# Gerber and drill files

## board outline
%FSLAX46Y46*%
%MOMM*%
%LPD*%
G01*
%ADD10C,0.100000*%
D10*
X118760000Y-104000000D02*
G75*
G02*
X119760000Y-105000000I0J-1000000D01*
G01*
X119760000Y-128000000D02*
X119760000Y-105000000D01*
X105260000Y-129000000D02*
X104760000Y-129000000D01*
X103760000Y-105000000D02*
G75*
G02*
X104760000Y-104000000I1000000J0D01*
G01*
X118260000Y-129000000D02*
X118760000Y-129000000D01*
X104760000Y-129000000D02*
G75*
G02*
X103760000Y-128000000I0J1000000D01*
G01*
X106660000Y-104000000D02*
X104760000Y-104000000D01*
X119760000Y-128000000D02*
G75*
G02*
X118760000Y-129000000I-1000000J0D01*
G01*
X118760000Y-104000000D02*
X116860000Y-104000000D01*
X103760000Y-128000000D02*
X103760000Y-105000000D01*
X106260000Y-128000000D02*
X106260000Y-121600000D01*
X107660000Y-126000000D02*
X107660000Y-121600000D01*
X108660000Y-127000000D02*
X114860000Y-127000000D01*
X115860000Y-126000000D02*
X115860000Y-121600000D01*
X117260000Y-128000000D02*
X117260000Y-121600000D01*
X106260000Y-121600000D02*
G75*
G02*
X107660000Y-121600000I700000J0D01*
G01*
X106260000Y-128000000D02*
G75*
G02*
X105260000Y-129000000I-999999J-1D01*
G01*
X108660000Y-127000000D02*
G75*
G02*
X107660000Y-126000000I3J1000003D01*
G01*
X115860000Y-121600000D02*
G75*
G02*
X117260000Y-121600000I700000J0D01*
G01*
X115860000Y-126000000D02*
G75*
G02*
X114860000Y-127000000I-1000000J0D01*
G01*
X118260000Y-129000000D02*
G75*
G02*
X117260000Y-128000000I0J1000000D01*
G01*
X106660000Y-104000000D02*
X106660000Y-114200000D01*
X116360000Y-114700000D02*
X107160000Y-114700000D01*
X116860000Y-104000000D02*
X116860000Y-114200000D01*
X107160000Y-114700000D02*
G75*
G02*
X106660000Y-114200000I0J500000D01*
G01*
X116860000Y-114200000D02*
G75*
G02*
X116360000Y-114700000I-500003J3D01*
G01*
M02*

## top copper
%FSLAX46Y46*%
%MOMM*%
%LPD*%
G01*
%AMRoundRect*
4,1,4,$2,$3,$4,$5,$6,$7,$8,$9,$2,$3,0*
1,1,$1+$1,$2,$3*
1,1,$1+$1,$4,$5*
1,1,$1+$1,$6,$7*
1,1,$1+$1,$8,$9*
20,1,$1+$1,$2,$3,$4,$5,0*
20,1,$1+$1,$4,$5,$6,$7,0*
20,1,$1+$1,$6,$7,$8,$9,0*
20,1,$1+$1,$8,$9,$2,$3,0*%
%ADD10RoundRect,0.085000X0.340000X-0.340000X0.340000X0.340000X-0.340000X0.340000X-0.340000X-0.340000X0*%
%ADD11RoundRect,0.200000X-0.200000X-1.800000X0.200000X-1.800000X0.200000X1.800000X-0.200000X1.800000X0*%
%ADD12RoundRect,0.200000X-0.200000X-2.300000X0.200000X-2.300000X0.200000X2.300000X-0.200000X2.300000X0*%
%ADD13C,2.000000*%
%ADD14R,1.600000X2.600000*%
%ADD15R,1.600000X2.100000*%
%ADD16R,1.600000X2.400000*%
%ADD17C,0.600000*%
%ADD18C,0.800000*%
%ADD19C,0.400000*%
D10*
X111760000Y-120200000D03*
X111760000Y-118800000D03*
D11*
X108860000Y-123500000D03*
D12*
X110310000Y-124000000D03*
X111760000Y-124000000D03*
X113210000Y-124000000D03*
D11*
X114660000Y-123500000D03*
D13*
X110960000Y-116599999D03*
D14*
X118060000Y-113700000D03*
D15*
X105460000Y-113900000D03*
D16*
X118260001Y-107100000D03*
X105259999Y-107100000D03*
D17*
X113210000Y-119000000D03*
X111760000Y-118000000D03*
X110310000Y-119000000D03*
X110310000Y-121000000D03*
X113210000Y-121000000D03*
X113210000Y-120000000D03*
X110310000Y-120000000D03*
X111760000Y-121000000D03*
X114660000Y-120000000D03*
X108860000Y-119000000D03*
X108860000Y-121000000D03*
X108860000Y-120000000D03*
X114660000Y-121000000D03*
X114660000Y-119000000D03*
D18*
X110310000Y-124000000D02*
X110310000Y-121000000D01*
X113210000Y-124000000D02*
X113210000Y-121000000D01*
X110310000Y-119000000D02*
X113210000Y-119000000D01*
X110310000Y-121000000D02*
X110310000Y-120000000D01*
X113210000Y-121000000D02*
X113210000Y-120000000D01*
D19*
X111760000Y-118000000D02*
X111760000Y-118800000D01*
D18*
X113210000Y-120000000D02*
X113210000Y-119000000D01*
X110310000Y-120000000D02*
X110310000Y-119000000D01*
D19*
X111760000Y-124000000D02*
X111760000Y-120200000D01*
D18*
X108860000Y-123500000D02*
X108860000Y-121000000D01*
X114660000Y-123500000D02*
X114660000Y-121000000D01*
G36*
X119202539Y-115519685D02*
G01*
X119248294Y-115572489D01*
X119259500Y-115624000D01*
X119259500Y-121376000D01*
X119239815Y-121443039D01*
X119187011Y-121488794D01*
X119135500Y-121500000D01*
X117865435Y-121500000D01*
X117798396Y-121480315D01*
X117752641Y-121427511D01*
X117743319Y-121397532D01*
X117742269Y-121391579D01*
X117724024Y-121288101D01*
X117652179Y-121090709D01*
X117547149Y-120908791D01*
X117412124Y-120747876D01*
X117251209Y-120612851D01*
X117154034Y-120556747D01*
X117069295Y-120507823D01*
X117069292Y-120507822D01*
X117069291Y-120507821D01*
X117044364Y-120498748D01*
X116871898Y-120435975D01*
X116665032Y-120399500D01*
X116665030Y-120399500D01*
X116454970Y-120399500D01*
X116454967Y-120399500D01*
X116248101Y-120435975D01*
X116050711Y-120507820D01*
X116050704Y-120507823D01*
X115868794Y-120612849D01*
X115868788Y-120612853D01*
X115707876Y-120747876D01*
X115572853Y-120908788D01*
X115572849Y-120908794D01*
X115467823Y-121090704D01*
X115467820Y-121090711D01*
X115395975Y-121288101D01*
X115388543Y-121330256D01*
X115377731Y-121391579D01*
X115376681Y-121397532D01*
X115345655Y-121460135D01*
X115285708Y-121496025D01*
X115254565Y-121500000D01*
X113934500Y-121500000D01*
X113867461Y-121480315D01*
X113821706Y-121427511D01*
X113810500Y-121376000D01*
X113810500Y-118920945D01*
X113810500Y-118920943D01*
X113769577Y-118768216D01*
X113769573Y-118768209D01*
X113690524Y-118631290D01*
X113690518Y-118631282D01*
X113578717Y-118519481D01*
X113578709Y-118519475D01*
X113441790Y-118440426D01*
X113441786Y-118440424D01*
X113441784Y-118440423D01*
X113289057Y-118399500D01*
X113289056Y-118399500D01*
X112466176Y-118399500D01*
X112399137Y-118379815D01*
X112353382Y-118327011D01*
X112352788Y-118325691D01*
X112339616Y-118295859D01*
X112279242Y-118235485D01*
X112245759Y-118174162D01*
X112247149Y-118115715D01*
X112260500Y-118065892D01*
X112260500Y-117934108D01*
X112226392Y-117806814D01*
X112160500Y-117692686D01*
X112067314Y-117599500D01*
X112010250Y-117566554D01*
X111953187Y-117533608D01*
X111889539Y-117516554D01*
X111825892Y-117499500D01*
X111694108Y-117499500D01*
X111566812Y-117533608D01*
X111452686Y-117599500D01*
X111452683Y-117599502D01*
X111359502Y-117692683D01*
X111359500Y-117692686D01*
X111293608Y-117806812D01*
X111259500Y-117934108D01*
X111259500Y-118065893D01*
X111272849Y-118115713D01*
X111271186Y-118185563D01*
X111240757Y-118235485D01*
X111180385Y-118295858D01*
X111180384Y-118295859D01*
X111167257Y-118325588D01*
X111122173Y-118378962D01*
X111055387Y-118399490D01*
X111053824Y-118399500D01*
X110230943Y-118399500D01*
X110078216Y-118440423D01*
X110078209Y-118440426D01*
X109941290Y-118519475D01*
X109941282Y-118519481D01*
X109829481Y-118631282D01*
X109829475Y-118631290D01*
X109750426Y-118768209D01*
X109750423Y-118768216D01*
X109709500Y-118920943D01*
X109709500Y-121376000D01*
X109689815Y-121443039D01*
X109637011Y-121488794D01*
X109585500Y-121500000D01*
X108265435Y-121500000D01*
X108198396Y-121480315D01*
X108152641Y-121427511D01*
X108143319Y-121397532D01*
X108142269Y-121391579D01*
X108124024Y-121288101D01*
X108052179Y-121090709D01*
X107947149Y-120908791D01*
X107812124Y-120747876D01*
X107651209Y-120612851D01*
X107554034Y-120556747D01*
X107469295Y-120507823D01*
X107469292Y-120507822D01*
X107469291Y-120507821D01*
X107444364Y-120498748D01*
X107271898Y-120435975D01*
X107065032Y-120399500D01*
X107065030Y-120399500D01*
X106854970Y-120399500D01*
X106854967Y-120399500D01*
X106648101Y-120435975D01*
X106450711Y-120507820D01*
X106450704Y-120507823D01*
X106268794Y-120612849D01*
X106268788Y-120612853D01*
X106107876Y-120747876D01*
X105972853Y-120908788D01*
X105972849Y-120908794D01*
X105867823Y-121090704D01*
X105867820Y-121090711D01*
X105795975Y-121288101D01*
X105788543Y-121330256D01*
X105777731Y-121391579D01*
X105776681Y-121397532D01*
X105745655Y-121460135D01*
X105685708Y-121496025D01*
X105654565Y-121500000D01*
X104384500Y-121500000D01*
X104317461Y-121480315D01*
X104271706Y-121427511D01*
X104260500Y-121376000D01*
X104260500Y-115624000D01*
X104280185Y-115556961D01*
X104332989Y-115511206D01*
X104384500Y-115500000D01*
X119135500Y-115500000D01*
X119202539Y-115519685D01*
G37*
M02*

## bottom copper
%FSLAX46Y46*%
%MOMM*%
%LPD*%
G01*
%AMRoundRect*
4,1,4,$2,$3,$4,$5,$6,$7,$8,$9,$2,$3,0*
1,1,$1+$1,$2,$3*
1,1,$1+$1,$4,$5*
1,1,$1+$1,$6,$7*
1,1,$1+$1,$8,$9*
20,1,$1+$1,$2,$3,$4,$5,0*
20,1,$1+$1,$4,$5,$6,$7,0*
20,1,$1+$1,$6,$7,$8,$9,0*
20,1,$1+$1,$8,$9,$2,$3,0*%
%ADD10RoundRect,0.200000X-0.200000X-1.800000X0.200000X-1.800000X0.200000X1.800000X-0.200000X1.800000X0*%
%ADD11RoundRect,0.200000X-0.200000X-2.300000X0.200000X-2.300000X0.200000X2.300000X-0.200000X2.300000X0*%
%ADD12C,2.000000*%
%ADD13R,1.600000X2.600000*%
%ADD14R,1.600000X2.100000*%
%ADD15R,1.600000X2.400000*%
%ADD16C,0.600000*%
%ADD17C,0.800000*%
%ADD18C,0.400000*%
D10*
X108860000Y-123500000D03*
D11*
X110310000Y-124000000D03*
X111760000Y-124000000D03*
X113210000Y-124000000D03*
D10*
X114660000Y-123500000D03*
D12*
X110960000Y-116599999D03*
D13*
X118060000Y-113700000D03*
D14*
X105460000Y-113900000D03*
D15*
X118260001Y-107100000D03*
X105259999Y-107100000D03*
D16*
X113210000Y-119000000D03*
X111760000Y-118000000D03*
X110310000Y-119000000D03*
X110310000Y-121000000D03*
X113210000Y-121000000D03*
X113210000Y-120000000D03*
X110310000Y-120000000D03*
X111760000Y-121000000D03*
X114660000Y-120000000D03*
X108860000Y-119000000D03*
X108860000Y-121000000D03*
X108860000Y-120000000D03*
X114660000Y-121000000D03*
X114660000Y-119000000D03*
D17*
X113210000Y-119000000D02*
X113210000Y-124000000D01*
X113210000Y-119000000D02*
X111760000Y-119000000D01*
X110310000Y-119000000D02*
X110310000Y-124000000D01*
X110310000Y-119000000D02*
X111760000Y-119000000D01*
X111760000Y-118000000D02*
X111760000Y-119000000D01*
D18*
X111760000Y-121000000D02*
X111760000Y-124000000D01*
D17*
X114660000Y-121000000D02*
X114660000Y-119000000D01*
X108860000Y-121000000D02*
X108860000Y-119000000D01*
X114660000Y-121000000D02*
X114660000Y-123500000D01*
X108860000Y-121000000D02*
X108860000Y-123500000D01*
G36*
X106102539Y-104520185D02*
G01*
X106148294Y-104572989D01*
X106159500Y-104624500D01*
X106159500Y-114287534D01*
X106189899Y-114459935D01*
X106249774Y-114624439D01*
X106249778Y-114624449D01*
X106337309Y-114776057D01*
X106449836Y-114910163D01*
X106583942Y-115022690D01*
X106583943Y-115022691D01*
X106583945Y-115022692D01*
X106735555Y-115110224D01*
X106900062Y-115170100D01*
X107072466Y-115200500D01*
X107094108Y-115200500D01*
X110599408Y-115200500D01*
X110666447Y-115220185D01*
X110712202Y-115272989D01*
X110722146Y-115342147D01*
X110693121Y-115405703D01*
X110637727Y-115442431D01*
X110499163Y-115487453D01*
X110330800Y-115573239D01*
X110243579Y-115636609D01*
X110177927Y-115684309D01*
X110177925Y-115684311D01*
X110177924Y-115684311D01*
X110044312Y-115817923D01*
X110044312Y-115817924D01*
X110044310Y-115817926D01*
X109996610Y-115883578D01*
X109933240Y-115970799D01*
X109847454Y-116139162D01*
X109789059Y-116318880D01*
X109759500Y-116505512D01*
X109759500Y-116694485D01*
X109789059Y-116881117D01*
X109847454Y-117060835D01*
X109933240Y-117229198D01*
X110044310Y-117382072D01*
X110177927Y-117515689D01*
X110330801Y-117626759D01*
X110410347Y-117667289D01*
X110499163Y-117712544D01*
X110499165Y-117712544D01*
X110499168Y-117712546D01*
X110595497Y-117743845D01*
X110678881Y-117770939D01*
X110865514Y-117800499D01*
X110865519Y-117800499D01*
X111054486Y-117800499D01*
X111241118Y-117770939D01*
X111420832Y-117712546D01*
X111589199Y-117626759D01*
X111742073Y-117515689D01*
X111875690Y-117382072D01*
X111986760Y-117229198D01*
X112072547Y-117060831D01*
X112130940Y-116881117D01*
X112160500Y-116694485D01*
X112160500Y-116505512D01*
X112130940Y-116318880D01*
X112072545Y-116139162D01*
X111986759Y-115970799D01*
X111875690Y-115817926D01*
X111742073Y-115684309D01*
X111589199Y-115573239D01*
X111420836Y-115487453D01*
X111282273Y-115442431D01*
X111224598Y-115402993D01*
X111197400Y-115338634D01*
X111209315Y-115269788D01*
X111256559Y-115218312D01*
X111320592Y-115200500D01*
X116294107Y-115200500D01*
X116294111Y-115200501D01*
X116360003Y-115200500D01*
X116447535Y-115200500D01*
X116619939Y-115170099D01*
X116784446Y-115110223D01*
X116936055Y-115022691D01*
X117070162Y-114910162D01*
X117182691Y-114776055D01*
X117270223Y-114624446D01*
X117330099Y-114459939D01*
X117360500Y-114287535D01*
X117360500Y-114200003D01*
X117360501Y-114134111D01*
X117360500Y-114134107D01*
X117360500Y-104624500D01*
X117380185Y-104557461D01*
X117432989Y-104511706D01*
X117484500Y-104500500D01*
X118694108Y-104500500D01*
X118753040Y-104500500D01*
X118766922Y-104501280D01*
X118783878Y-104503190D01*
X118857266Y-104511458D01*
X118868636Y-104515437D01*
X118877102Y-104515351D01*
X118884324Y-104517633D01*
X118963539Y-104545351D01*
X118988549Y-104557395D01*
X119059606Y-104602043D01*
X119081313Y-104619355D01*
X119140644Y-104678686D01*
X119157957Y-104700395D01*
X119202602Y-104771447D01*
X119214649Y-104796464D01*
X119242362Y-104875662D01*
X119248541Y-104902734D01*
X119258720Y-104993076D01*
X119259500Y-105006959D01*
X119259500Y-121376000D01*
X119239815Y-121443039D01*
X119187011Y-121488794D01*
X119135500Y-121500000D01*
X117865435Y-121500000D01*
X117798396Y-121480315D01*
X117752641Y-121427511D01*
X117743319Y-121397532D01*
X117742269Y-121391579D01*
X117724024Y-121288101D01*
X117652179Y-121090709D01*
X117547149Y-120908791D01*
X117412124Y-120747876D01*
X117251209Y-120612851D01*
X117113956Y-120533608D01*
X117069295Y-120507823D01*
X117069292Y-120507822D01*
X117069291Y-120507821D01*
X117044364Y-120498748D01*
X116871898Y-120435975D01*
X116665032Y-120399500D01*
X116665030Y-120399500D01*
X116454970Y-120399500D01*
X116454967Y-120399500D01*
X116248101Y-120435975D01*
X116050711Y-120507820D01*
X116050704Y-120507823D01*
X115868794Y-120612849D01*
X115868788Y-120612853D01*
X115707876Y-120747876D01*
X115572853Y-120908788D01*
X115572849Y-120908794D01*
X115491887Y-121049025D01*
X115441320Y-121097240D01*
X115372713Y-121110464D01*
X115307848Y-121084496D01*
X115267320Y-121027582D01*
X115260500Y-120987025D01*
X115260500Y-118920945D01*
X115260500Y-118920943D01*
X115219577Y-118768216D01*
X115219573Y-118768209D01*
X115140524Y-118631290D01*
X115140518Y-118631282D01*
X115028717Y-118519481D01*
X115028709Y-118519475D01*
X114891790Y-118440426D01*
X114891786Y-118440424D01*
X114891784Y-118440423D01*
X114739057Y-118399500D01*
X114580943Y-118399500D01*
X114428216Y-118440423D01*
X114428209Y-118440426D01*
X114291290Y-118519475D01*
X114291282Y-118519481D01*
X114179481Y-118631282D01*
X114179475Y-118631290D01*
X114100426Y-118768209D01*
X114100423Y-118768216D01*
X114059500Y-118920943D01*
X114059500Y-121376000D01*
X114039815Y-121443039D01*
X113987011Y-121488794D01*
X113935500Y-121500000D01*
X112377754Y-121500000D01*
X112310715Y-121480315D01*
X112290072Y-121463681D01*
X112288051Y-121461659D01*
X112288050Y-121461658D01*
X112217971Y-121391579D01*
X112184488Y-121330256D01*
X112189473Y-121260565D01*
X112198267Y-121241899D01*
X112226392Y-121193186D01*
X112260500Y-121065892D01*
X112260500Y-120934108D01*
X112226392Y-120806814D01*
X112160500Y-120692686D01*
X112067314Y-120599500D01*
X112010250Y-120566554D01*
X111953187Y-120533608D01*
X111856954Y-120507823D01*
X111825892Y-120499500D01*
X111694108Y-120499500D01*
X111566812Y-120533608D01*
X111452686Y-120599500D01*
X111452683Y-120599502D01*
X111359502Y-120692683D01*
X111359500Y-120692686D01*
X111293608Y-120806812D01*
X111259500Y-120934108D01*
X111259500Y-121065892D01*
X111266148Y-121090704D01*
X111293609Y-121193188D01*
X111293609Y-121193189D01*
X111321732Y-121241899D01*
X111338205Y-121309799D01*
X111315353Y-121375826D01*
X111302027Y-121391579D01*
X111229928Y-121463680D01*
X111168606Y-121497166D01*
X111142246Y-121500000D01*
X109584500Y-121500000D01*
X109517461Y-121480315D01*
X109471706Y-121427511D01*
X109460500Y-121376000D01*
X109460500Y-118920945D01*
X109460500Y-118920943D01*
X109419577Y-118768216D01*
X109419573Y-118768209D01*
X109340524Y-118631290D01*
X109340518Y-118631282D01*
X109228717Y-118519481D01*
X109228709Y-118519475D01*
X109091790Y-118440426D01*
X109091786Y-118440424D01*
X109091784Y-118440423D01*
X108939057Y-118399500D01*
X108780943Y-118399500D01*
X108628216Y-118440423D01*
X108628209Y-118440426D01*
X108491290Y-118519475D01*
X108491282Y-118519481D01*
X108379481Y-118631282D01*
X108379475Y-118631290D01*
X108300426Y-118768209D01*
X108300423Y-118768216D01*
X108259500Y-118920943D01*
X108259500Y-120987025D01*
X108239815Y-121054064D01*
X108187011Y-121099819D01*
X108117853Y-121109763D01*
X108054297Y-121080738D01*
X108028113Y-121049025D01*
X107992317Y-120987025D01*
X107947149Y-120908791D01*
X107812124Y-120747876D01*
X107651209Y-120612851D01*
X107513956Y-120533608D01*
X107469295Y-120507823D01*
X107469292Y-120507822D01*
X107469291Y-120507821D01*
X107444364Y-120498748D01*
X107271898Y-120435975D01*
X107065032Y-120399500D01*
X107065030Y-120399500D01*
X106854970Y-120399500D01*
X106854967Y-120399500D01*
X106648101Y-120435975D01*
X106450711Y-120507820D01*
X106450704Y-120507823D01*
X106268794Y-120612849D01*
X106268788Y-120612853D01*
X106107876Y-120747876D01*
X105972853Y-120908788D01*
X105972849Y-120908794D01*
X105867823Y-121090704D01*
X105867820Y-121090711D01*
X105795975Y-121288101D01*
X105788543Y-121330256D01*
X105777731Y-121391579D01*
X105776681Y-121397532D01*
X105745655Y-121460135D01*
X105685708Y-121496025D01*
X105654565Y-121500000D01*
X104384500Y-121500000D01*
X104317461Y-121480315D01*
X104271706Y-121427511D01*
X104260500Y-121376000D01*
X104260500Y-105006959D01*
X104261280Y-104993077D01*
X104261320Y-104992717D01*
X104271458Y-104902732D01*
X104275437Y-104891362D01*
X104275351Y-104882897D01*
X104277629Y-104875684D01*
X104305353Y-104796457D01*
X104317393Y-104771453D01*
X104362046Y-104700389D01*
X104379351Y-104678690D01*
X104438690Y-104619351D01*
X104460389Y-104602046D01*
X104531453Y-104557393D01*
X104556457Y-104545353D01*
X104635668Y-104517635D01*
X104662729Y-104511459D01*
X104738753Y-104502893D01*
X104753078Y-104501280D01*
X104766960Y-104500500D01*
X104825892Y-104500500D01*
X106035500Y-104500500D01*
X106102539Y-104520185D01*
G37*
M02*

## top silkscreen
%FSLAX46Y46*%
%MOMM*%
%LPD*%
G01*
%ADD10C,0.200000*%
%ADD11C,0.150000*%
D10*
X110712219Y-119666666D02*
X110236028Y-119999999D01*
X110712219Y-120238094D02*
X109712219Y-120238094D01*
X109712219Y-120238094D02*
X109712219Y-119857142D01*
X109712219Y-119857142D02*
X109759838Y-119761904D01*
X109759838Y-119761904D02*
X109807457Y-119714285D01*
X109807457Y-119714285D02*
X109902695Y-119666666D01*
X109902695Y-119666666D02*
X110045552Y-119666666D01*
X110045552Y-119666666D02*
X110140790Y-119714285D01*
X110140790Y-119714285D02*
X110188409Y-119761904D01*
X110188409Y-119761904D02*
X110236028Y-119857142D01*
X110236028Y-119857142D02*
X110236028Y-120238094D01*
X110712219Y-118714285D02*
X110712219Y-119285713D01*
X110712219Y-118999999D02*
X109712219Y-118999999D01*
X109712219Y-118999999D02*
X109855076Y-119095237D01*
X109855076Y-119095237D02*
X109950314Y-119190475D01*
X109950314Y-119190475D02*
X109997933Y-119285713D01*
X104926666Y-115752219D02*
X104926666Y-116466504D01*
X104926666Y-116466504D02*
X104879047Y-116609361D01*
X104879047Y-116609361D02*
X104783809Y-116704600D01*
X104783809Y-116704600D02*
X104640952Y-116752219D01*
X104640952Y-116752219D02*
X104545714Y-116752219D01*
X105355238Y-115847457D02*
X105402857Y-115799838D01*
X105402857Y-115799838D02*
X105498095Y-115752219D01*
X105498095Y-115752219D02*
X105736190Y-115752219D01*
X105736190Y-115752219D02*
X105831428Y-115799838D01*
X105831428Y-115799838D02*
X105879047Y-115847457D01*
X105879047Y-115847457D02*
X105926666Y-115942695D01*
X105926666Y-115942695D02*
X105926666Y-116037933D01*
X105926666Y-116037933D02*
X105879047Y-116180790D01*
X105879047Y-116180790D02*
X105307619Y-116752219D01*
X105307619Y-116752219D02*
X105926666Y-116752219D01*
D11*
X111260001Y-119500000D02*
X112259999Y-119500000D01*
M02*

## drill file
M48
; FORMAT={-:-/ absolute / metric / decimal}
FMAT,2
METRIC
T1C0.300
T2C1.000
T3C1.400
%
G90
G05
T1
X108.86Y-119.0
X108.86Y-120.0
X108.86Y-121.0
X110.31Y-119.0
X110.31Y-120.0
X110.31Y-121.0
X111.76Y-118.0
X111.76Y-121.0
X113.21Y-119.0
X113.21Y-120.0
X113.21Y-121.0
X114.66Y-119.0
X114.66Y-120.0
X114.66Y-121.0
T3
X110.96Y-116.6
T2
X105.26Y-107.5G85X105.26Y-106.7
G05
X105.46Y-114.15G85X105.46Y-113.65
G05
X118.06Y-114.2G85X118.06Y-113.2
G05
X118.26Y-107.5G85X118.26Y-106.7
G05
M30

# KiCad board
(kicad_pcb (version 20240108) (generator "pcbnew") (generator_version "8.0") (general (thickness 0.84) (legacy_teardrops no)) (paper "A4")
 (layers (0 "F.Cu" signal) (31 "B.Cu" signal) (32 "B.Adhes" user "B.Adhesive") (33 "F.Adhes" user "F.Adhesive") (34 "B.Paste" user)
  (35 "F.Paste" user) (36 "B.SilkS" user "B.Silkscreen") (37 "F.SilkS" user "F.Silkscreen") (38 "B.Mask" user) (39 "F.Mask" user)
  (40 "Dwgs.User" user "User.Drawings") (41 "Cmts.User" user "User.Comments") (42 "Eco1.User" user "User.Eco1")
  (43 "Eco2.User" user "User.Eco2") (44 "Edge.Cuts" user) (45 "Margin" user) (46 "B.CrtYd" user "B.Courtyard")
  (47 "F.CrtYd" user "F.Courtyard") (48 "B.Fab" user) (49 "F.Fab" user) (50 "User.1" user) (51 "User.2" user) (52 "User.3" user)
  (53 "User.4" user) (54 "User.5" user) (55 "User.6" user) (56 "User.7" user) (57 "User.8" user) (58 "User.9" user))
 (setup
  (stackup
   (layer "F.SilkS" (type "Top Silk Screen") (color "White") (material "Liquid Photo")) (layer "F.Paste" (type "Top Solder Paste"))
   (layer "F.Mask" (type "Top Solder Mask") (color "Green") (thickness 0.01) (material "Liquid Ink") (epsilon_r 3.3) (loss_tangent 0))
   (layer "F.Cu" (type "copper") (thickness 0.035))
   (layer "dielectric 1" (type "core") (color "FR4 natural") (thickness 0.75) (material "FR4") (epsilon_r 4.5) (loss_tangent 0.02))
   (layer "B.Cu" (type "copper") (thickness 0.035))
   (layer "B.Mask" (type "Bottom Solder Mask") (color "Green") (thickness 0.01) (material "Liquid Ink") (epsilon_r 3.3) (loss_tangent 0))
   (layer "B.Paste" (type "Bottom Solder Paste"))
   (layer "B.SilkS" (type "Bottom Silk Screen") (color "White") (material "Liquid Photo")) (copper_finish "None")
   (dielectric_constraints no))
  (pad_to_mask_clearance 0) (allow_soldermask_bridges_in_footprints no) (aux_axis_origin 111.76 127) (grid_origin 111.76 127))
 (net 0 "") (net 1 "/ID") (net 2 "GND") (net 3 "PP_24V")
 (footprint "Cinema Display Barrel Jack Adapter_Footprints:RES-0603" (layer "F.Cu") (at 111.76 119.5 90)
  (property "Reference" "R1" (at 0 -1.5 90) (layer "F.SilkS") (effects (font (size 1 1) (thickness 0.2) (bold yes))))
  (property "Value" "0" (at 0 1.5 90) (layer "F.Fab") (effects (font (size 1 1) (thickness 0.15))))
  (fp_line (start 0 -0.499999) (end 0 0.499999) (stroke (width 0.15) (type default)) (layer "F.SilkS"))
  (pad "1" smd roundrect (at -0.7 0 90) (size 0.85 0.85) (layers "F.Cu" "F.Paste" "F.Mask") (roundrect_rratio 0.1) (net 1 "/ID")
   (solder_paste_margin_ratio -0.05))
  (pad "2" smd roundrect (at 0.7 0 90) (size 0.85 0.85) (layers "F.Cu" "F.Paste" "F.Mask") (roundrect_rratio 0.1) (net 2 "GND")
   (solder_paste_margin_ratio -0.05)))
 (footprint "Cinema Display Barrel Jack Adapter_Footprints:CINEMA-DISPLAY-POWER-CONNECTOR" (layer "F.Cu") (at 111.76 127)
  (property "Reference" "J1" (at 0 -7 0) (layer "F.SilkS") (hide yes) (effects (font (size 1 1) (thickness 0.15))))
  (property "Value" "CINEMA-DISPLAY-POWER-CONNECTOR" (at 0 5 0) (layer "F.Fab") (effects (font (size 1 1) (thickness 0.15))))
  (fp_line (start -5.5 1) (end -5.5 -5.4) (stroke (width 0.1) (type default)) (layer "Edge.Cuts"))
  (fp_line (start -4.1 -1) (end -4.1 -5.4) (stroke (width 0.1) (type default)) (layer "Edge.Cuts"))
  (fp_line (start -3.1 0) (end 3.1 0) (stroke (width 0.1) (type default)) (layer "Edge.Cuts"))
  (fp_line (start 4.1 -1) (end 4.1 -5.4) (stroke (width 0.1) (type default)) (layer "Edge.Cuts"))
  (fp_line (start 5.5 1) (end 5.5 -5.4) (stroke (width 0.1) (type default)) (layer "Edge.Cuts"))
  (fp_arc (start -5.5 -5.4) (mid -4.8 -6.1) (end -4.1 -5.4) (stroke (width 0.1) (type default)) (layer "Edge.Cuts"))
  (fp_arc (start -5.5 1) (mid -5.792893 1.707107) (end -6.5 2) (stroke (width 0.1) (type default)) (layer "Edge.Cuts"))
  (fp_arc (start -3.1 0) (mid -3.807106 -0.292894) (end -4.1 -1) (stroke (width 0.1) (type default)) (layer "Edge.Cuts"))
  (fp_arc (start 4.1 -5.4) (mid 4.8 -6.1) (end 5.5 -5.4) (stroke (width 0.1) (type default)) (layer "Edge.Cuts"))
  (fp_arc (start 4.1 -1) (mid 3.807107 -0.292893) (end 3.1 0) (stroke (width 0.1) (type default)) (layer "Edge.Cuts"))
  (fp_arc (start 6.5 2) (mid 5.792893 1.707107) (end 5.5 1) (stroke (width 0.1) (type default)) (layer "Edge.Cuts"))
  (pad "1" smd roundrect (at -2.9 -3.5) (size 0.8 4) (layers "F.Cu" "F.Mask") (roundrect_rratio 0.25) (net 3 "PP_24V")
   (thermal_bridge_angle 45))
  (pad "1" smd roundrect (at -2.9 -3.5) (size 0.8 4) (layers "B.Cu" "B.Mask") (roundrect_rratio 0.25) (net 3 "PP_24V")
   (thermal_bridge_angle 45))
  (pad "2" smd roundrect (at -1.45 -3) (size 0.8 5) (layers "F.Cu" "F.Mask") (roundrect_rratio 0.25) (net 2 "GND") (thermal_bridge_angle 45))
  (pad "2" smd roundrect (at -1.45 -3) (size 0.8 5) (layers "B.Cu" "B.Mask") (roundrect_rratio 0.25) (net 2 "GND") (thermal_bridge_angle 45))
  (pad "3" smd roundrect (at 0 -3) (size 0.8 5) (layers "F.Cu" "F.Mask") (roundrect_rratio 0.25) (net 1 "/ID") (thermal_bridge_angle 45))
  (pad "3" smd roundrect (at 0 -3) (size 0.8 5) (layers "B.Cu" "B.Mask") (roundrect_rratio 0.25) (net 1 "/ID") (thermal_bridge_angle 45))
  (pad "4" smd roundrect (at 1.45 -3) (size 0.8 5) (layers "F.Cu" "F.Mask") (roundrect_rratio 0.25) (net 2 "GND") (thermal_bridge_angle 45))
  (pad "4" smd roundrect (at 1.45 -3) (size 0.8 5) (layers "B.Cu" "B.Mask") (roundrect_rratio 0.25) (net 2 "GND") (thermal_bridge_angle 45))
  (pad "5" smd roundrect (at 2.9 -3.5) (size 0.8 4) (layers "F.Cu" "F.Mask") (roundrect_rratio 0.25) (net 3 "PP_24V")
   (thermal_bridge_angle 45))
  (pad "5" smd roundrect (at 2.9 -3.5) (size 0.8 4) (layers "B.Cu" "B.Mask") (roundrect_rratio 0.25) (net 3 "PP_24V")
   (thermal_bridge_angle 45))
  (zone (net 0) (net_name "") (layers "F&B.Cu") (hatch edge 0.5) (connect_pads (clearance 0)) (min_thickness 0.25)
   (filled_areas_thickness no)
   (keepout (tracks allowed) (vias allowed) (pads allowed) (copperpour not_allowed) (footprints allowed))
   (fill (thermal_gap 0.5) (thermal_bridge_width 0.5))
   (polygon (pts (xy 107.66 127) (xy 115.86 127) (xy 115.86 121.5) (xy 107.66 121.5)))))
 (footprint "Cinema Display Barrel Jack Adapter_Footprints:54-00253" (layer "F.Cu") (at 111.76 108.8 180)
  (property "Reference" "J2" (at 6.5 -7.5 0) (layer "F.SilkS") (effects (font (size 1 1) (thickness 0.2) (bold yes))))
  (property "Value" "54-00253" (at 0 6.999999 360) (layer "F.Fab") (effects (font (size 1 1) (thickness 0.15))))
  (fp_line (start 5.1 4.8) (end 5.1 -5.4) (stroke (width 0.1) (type default)) (layer "Edge.Cuts"))
  (fp_line (start -4.6 -5.9) (end 4.6 -5.9) (stroke (width 0.1) (type default)) (layer "Edge.Cuts"))
  (fp_line (start -5.1 4.8) (end -5.1 -5.4) (stroke (width 0.1) (type default)) (layer "Edge.Cuts"))
  (fp_arc (start 4.6 -5.9) (mid 4.953553 -5.753553) (end 5.1 -5.4) (stroke (width 0.1) (type default)) (layer "Edge.Cuts"))
  (fp_arc (start -5.1 -5.4) (mid -4.953553 -5.753552) (end -4.6 -5.9) (stroke (width 0.1) (type default)) (layer "Edge.Cuts"))
  (pad "A" thru_hole circle (at 0.8 -7.799999 180) (size 2 2) (drill 1.4) (layers "*.Cu" "*.Mask") (remove_unused_layers no)
   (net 3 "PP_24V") (zone_connect 2) (thermal_bridge_angle 90))
  (pad "B" thru_hole rect (at -6.3 -4.9 180) (size 1.6 2.6) (drill oval 1 2) (layers "*.Cu" "*.Mask") (remove_unused_layers no)
   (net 2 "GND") (zone_connect 2))
  (pad "C" thru_hole rect (at 6.3 -5.1 180) (size 1.6 2.1) (drill oval 1 1.5) (layers "*.Cu" "*.Mask") (remove_unused_layers no)
   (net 2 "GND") (zone_connect 2))
  (pad "D" thru_hole rect (at -6.500001 1.7 180) (size 1.6 2.4) (drill oval 1 1.8) (layers "*.Cu" "*.Mask") (remove_unused_layers no)
   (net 2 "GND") (zone_connect 2))
  (pad "D" thru_hole rect (at 6.500001 1.7 180) (size 1.6 2.4) (drill oval 1 1.8) (layers "*.Cu" "*.Mask") (remove_unused_layers no)
   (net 2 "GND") (zone_connect 2)))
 (gr_arc (start 118.76 104) (mid 119.467107 104.292893) (end 119.76 105) (stroke (width 0.1) (type default)) (layer "Edge.Cuts"))
 (gr_line (start 119.76 128) (end 119.76 105) (stroke (width 0.1) (type default)) (layer "Edge.Cuts"))
 (gr_line (start 105.26 129) (end 104.76 129) (stroke (width 0.1) (type default)) (layer "Edge.Cuts"))
 (gr_arc (start 103.76 105) (mid 104.052893 104.292893) (end 104.76 104) (stroke (width 0.1) (type default)) (layer "Edge.Cuts"))
 (gr_line (start 118.26 129) (end 118.76 129) (stroke (width 0.1) (type default)) (layer "Edge.Cuts"))
 (gr_arc (start 104.76 129) (mid 104.052893 128.707107) (end 103.76 128) (stroke (width 0.1) (type default)) (layer "Edge.Cuts"))
 (gr_line (start 106.66 104) (end 104.76 104) (stroke (width 0.1) (type default)) (layer "Edge.Cuts"))
 (gr_arc (start 119.76 128) (mid 119.467107 128.707107) (end 118.76 129) (stroke (width 0.1) (type default)) (layer "Edge.Cuts"))
 (gr_line (start 118.76 104) (end 116.86 104) (stroke (width 0.1) (type default)) (layer "Edge.Cuts"))
 (gr_line (start 103.76 128) (end 103.76 105) (stroke (width 0.1) (type default)) (layer "Edge.Cuts"))
 (segment (start 110.31 124) (end 110.31 121) (width 0.8) (layer "F.Cu") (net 2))
 (segment (start 113.21 124) (end 113.21 121) (width 0.8) (layer "F.Cu") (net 2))
 (segment (start 110.31 119) (end 113.21 119) (width 0.8) (layer "F.Cu") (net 2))
 (segment (start 110.31 121) (end 110.31 120) (width 0.8) (layer "F.Cu") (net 2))
 (segment (start 113.21 121) (end 113.21 120) (width 0.8) (layer "F.Cu") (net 2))
 (segment (start 111.76 118) (end 111.76 118.8) (width 0.4) (layer "F.Cu") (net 2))
 (segment (start 113.21 120) (end 113.21 119) (width 0.8) (layer "F.Cu") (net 2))
 (segment (start 110.31 120) (end 110.31 119) (width 0.8) (layer "F.Cu") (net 2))
 (via (at 113.21 119) (size 0.6) (drill 0.3) (layers "F.Cu" "B.Cu") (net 2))
 (via (at 111.76 118) (size 0.6) (drill 0.3) (layers "F.Cu" "B.Cu") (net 2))
 (via (at 110.31 119) (size 0.6) (drill 0.3) (layers "F.Cu" "B.Cu") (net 2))
 (via (at 110.31 121) (size 0.6) (drill 0.3) (layers "F.Cu" "B.Cu") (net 2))
 (via (at 113.21 121) (size 0.6) (drill 0.3) (layers "F.Cu" "B.Cu") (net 2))
 (via (at 113.21 120) (size 0.6) (drill 0.3) (layers "F.Cu" "B.Cu") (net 2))
 (via (at 110.31 120) (size 0.6) (drill 0.3) (layers "F.Cu" "B.Cu") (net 2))
 (segment (start 113.21 119) (end 113.21 124) (width 0.8) (layer "B.Cu") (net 2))
 (segment (start 113.21 119) (end 111.76 119) (width 0.8) (layer "B.Cu") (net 2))
 (segment (start 110.31 119) (end 110.31 124) (width 0.8) (layer "B.Cu") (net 2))
 (segment (start 110.31 119) (end 111.76 119) (width 0.8) (layer "B.Cu") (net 2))
 (segment (start 111.76 118) (end 111.76 119) (width 0.8) (layer "B.Cu") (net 2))
 (segment (start 111.76 124) (end 111.76 120.2) (width 0.4) (layer "F.Cu") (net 1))
 (via (at 111.76 121) (size 0.6) (drill 0.3) (layers "F.Cu" "B.Cu") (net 1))
 (segment (start 111.76 121) (end 111.76 124) (width 0.4) (layer "B.Cu") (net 1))
 (segment (start 108.86 123.5) (end 108.86 121) (width 0.8) (layer "F.Cu") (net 3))
 (segment (start 114.66 123.5) (end 114.66 121) (width 0.8) (layer "F.Cu") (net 3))
 (via (at 114.66 120) (size 0.6) (drill 0.3) (layers "F.Cu" "B.Cu") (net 3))
 (via (at 108.86 119) (size 0.6) (drill 0.3) (layers "F.Cu" "B.Cu") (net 3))
 (via (at 108.86 121) (size 0.6) (drill 0.3) (layers "F.Cu" "B.Cu") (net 3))
 (via (at 108.86 120) (size 0.6) (drill 0.3) (layers "F.Cu" "B.Cu") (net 3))
 (via (at 114.66 121) (size 0.6) (drill 0.3) (layers "F.Cu" "B.Cu") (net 3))
 (via (at 114.66 119) (size 0.6) (drill 0.3) (layers "F.Cu" "B.Cu") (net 3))
 (segment (start 114.66 121) (end 114.66 119) (width 0.8) (layer "B.Cu") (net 3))
 (segment (start 108.86 121) (end 108.86 119) (width 0.8) (layer "B.Cu") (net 3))
 (segment (start 114.66 121) (end 114.66 123.5) (width 0.8) (layer "B.Cu") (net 3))
 (segment (start 108.86 121) (end 108.86 123.5) (width 0.8) (layer "B.Cu") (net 3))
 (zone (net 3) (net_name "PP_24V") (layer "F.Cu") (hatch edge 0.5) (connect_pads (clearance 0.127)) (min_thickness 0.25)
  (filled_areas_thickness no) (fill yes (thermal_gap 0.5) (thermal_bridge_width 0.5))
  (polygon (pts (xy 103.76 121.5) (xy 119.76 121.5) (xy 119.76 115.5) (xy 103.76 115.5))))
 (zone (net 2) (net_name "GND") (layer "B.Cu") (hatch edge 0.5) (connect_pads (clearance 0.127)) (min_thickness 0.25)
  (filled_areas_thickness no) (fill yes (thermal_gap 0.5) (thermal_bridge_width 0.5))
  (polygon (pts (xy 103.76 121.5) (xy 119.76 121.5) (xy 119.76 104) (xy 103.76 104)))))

